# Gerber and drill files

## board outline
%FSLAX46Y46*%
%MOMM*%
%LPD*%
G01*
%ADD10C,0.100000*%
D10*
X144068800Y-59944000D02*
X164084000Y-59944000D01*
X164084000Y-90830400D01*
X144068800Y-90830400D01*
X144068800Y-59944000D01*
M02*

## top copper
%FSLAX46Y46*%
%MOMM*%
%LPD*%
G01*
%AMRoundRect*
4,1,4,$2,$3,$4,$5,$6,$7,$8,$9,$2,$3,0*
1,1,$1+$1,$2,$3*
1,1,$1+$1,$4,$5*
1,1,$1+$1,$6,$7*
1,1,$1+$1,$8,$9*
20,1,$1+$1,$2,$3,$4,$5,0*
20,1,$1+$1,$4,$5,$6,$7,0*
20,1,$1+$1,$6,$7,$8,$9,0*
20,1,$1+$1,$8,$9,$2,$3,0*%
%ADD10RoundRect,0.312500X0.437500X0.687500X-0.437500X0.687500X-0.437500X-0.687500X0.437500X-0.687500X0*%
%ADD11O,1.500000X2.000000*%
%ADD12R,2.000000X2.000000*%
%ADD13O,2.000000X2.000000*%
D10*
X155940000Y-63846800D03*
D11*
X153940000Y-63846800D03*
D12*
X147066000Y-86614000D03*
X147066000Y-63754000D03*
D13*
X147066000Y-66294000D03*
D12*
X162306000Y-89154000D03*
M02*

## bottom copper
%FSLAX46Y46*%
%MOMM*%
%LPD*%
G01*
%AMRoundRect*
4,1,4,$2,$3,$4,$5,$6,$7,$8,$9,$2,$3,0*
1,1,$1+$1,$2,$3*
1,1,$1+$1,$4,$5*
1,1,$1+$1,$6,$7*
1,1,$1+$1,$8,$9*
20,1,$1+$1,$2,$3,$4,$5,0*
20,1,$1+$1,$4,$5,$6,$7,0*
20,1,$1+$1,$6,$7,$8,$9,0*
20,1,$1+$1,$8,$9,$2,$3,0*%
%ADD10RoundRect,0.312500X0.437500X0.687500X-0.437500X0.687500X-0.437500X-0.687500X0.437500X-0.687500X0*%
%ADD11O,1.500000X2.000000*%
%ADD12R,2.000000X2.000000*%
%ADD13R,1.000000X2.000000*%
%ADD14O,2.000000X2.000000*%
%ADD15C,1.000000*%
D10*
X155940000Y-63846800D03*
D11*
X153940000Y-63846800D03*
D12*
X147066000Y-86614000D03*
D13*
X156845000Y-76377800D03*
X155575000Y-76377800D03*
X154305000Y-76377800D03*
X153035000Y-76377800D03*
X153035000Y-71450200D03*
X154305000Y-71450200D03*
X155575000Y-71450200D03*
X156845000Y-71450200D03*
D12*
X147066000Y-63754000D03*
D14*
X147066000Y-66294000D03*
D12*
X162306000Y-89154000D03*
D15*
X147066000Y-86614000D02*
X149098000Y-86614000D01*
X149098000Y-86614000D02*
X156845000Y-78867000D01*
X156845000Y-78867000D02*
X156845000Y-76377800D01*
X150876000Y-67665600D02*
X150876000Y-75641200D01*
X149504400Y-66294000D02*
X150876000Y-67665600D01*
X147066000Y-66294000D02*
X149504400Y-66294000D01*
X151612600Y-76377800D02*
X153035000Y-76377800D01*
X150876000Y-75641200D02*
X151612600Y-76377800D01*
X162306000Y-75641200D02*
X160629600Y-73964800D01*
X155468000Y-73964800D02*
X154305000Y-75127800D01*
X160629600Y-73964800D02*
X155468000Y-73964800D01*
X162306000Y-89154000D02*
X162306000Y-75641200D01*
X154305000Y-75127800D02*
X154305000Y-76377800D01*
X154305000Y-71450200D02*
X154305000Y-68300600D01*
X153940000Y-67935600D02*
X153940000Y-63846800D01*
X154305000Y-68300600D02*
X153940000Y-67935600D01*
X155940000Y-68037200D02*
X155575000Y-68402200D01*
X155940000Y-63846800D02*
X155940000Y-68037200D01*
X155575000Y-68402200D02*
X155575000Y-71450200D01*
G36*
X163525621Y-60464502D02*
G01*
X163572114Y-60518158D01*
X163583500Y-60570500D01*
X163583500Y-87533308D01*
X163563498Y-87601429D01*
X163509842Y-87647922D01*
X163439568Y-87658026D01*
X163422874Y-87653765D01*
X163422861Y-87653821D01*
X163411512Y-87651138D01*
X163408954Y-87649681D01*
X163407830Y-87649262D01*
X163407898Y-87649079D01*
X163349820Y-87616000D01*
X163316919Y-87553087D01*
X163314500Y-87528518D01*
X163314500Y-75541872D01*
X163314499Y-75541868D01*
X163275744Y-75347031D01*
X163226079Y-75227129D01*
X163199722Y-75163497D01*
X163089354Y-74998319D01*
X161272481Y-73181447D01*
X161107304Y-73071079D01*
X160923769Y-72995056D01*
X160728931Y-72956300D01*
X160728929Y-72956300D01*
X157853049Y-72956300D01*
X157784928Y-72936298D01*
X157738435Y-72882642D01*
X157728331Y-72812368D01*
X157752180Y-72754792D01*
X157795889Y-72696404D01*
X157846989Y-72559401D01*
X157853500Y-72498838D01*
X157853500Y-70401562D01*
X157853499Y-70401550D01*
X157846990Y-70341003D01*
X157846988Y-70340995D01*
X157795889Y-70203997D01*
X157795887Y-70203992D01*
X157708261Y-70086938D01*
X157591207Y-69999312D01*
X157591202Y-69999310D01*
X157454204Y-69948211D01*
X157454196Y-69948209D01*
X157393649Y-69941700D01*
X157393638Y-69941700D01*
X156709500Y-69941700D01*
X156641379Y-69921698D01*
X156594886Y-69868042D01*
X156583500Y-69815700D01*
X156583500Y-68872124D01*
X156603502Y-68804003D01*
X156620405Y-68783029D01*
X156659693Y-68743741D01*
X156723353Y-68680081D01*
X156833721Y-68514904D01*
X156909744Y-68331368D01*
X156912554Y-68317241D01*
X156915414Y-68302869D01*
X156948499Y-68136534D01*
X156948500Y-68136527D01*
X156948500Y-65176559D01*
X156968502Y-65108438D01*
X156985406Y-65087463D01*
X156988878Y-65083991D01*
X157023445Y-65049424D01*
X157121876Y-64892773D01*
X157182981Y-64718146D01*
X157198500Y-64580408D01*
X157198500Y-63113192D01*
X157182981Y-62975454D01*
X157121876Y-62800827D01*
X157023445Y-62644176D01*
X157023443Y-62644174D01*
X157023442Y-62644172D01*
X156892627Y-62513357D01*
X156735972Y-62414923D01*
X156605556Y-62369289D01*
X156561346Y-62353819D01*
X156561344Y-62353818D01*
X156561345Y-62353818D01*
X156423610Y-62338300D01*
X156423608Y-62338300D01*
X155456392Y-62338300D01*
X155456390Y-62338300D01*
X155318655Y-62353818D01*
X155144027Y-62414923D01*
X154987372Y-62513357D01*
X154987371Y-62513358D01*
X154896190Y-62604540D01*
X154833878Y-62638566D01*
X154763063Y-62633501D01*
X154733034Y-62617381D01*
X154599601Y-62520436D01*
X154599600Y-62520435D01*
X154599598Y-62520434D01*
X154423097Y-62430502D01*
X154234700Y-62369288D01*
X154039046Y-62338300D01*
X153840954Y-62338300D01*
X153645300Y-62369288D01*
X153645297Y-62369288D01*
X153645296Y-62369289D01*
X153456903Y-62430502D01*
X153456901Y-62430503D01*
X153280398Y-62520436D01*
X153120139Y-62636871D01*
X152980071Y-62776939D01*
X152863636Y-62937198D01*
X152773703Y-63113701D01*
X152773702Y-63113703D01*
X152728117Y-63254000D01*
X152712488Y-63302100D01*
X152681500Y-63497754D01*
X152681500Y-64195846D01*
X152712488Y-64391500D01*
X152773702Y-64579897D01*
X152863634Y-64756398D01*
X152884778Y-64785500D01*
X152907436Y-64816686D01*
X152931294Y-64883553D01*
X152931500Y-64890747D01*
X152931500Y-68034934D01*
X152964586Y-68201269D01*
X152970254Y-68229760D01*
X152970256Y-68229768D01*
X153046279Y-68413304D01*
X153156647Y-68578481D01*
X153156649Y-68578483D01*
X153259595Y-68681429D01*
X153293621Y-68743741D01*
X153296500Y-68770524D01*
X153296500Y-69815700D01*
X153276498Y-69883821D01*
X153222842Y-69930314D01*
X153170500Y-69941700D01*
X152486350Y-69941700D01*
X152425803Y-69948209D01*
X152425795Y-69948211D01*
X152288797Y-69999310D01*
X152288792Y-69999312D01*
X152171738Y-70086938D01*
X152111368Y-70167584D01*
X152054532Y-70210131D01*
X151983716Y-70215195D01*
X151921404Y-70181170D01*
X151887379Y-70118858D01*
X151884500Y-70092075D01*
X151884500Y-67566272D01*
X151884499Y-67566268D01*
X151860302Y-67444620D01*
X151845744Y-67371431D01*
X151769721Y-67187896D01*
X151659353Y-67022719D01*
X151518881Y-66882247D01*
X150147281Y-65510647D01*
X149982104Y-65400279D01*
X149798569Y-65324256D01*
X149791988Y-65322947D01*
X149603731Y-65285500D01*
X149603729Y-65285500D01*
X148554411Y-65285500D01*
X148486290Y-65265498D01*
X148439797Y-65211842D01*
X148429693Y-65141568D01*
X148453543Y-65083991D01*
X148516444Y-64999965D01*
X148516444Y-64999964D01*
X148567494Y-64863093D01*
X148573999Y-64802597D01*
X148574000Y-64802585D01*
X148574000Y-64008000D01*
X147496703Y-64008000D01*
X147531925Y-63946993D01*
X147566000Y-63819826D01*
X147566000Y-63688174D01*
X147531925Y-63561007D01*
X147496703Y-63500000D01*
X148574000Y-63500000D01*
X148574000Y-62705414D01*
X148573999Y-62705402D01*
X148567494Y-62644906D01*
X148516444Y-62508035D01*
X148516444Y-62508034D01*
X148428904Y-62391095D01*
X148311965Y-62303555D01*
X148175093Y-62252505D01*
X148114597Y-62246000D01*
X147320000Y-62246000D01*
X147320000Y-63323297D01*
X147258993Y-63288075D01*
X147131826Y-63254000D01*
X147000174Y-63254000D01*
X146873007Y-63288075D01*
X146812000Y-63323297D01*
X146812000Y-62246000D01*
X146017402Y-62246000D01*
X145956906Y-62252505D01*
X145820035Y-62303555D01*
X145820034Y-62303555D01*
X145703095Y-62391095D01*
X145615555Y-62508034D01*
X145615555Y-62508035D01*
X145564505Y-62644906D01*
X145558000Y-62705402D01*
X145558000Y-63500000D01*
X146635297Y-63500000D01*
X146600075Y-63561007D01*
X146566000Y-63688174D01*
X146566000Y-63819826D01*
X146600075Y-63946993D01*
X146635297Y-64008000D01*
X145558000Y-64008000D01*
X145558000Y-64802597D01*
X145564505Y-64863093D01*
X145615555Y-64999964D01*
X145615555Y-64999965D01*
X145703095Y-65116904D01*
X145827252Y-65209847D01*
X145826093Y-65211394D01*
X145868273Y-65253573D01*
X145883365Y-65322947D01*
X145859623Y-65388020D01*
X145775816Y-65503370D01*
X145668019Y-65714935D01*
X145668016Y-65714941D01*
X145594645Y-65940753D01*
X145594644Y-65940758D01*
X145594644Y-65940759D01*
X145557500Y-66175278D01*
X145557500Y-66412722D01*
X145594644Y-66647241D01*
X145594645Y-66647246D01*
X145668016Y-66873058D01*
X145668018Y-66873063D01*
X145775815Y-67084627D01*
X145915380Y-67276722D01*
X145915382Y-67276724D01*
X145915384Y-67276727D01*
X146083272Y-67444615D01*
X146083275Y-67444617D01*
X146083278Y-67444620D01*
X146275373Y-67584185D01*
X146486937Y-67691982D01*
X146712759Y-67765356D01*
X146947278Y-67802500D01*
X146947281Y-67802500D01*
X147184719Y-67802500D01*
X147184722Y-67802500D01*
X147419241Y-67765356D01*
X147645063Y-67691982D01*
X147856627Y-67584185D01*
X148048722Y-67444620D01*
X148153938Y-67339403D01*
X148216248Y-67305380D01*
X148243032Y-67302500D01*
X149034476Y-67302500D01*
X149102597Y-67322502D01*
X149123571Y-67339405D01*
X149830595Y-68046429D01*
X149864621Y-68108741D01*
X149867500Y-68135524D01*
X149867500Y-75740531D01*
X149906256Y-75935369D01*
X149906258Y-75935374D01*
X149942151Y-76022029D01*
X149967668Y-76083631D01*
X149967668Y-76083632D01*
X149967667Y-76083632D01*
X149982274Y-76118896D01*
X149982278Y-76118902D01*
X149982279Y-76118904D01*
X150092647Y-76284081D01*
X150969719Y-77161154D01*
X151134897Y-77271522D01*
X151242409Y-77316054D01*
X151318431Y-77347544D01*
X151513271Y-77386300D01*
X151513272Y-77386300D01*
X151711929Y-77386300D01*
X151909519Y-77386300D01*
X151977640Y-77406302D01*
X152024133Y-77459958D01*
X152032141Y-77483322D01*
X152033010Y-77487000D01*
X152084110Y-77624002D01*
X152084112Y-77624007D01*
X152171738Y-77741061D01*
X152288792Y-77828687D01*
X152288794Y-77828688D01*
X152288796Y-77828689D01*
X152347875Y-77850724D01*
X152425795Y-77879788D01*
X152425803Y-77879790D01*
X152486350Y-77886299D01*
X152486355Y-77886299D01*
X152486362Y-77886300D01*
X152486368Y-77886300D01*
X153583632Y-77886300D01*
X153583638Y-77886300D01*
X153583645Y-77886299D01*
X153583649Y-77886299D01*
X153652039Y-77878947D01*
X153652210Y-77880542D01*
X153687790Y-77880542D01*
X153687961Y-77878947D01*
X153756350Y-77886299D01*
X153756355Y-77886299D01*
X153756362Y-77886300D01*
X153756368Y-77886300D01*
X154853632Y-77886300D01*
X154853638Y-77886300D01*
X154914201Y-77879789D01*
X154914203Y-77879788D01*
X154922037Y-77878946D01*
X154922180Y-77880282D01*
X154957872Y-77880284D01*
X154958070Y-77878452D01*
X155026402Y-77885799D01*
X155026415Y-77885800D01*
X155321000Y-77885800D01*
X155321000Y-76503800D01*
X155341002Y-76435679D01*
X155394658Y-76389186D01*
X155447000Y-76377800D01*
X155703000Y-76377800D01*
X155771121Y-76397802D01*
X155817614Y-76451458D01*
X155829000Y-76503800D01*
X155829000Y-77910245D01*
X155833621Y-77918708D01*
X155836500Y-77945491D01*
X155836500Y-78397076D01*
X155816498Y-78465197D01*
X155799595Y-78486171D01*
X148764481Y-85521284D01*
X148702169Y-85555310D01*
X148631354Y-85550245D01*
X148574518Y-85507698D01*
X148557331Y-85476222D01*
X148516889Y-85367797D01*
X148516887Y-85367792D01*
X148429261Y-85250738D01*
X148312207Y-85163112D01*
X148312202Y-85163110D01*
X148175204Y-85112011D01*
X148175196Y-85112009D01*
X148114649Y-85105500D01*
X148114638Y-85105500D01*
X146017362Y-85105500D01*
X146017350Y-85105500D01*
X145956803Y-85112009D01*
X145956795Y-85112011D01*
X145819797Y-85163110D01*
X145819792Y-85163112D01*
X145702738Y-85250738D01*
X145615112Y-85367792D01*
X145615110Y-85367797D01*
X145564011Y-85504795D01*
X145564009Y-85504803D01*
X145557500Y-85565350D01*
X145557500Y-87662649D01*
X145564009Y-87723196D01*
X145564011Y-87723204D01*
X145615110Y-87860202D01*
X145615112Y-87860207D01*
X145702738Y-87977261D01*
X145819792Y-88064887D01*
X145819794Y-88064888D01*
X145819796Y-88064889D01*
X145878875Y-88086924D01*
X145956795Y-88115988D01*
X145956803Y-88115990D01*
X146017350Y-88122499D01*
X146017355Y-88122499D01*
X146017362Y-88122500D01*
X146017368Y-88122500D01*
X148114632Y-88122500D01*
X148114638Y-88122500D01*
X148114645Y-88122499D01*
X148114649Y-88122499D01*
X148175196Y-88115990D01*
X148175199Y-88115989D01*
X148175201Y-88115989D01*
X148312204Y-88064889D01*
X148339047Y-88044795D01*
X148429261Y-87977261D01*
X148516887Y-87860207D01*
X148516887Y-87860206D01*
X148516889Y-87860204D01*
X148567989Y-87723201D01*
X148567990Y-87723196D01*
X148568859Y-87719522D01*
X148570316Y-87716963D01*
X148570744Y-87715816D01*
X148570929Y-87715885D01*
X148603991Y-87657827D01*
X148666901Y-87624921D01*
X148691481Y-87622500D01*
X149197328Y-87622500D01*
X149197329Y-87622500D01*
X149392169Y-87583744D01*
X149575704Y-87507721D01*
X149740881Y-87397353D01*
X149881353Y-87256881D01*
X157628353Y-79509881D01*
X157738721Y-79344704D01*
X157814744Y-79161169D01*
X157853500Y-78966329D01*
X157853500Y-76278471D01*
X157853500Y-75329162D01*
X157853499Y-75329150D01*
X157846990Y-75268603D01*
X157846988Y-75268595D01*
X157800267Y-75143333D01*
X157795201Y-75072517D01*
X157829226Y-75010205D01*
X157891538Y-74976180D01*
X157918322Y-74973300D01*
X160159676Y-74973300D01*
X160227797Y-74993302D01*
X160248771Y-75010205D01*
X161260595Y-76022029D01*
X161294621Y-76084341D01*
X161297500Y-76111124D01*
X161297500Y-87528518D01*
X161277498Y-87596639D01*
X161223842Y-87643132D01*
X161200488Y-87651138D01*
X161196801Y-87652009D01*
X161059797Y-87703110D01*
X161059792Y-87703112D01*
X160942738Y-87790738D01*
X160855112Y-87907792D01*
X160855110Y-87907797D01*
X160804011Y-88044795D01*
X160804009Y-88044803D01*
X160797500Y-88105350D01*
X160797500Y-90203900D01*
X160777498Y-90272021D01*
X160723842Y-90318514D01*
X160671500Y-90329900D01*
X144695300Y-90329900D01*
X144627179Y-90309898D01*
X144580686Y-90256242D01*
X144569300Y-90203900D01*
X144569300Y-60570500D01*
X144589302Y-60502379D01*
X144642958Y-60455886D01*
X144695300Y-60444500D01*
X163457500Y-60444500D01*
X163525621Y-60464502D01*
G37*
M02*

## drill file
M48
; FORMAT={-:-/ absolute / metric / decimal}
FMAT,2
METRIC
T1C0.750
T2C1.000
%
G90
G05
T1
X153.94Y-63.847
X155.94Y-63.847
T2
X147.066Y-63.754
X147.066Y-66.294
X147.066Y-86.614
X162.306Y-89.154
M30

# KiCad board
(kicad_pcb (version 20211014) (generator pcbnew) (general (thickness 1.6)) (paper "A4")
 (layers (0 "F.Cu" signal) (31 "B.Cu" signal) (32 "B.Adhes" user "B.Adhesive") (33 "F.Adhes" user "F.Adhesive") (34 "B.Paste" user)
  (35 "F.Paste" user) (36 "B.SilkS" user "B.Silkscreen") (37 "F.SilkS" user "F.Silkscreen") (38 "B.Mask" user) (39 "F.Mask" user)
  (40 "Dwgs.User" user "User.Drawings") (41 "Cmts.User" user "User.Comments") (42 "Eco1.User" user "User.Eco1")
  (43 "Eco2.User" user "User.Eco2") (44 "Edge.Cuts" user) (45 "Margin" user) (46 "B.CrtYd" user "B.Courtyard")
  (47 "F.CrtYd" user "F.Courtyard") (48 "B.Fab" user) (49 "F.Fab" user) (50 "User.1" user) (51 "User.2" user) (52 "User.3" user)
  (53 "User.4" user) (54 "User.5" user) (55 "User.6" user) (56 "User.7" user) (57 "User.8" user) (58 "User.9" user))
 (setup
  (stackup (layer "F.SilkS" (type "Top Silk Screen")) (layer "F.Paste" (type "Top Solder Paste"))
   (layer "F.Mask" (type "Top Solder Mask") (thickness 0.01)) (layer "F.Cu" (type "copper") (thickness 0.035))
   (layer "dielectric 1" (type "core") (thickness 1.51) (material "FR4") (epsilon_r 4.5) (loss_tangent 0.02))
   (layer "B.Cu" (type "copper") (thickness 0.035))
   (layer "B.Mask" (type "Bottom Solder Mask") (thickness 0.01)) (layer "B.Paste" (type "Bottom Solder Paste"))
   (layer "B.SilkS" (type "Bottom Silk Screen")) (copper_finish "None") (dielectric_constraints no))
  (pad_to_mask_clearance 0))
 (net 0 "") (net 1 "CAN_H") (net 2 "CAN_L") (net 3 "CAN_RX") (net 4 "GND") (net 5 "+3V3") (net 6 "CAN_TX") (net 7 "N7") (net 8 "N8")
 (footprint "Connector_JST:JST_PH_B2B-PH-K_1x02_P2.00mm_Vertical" (layer "F.Cu") (at 155.94 63.8468 180)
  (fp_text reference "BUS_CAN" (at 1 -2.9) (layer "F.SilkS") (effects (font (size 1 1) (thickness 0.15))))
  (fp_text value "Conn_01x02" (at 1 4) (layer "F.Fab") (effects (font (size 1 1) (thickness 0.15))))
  (pad "1" thru_hole roundrect locked (at 0 0 180) (size 1.5 2) (drill 0.75) (layers *.Cu *.Mask) (roundrect_rratio 0.208333)
   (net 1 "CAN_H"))
  (pad "2" thru_hole oval locked (at 2 0 180) (size 1.5 2) (drill 0.75) (layers *.Cu *.Mask) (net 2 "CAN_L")))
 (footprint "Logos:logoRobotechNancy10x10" (layer "F.Cu") (at 154.432 74.93)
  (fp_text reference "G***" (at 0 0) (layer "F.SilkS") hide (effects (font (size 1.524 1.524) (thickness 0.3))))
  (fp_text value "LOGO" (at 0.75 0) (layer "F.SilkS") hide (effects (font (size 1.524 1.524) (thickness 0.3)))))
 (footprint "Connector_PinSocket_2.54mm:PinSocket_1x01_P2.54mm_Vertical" (layer "B.Cu") (at 147.066 86.614 180)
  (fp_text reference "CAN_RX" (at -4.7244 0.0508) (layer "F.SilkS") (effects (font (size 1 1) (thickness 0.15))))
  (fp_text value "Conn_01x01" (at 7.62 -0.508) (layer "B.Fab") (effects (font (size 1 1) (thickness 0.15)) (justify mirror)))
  (pad "1" thru_hole rect locked (at 0 0 180) (size 2 2) (drill 1) (layers *.Cu *.Mask) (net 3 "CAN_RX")))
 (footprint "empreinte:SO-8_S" (layer "B.Cu") (at 154.94 73.914 90)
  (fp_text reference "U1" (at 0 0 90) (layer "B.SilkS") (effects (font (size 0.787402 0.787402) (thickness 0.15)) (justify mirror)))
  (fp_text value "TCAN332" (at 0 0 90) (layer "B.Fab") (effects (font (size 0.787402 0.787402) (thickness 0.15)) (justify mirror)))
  (pad "1" smd rect locked (at -2.4638 1.905 90) (size 2 1) (layers "B.Cu" "B.Paste" "B.Mask") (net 3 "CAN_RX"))
  (pad "2" smd rect locked (at -2.4638 0.635 90) (size 2 1) (layers "B.Cu" "B.Paste" "B.Mask") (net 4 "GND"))
  (pad "3" smd rect locked (at -2.4638 -0.635 90) (size 2 1) (layers "B.Cu" "B.Paste" "B.Mask") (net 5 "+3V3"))
  (pad "4" smd rect locked (at -2.4638 -1.905 90) (size 2 1) (layers "B.Cu" "B.Paste" "B.Mask") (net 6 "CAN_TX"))
  (pad "5" smd rect locked (at 2.4638 -1.905 90) (size 2 1) (layers "B.Cu" "B.Paste" "B.Mask") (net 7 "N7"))
  (pad "6" smd rect locked (at 2.4638 -0.635 90) (size 2 1) (layers "B.Cu" "B.Paste" "B.Mask") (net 2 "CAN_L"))
  (pad "7" smd rect locked (at 2.4638 0.635 90) (size 2 1) (layers "B.Cu" "B.Paste" "B.Mask") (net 1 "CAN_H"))
  (pad "8" smd rect locked (at 2.4638 1.905 90) (size 2 1) (layers "B.Cu" "B.Paste" "B.Mask") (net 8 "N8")))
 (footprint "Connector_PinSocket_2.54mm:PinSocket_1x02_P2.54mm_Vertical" (layer "B.Cu") (at 147.066 63.754 180)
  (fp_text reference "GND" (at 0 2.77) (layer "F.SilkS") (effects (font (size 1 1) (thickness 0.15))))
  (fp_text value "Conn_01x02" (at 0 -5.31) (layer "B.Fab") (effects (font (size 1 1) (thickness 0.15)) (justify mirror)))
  (pad "1" thru_hole rect locked (at 0 0 180) (size 2 2) (drill 1) (layers *.Cu *.Mask) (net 4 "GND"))
  (pad "2" thru_hole oval locked (at 0 -2.54 180) (size 2 2) (drill 1) (layers *.Cu *.Mask) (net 6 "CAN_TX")))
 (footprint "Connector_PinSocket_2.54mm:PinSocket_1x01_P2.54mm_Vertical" (layer "B.Cu") (at 162.306 89.154 180)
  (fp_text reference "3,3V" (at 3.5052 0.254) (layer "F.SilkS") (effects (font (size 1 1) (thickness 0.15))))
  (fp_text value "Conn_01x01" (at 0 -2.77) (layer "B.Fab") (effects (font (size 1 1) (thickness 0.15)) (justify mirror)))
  (pad "1" thru_hole rect locked (at 0 0 180) (size 2 2) (drill 1) (layers *.Cu *.Mask) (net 5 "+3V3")))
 (gr_rect (start 144.0688 59.944) (end 164.084 90.8304) (layer "Edge.Cuts") (width 0.1) (fill none))
 (segment (start 147.066 86.614) (end 149.098 86.614) (width 1) (layer "B.Cu") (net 3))
 (segment (start 149.098 86.614) (end 156.845 78.867) (width 1) (layer "B.Cu") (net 3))
 (segment (start 156.845 78.867) (end 156.845 76.3778) (width 1) (layer "B.Cu") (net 3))
 (segment (start 150.876 67.6656) (end 150.876 75.6412) (width 1) (layer "B.Cu") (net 6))
 (segment (start 149.5044 66.294) (end 150.876 67.6656) (width 1) (layer "B.Cu") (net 6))
 (segment (start 147.066 66.294) (end 149.5044 66.294) (width 1) (layer "B.Cu") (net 6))
 (segment (start 151.6126 76.3778) (end 153.035 76.3778) (width 1) (layer "B.Cu") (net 6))
 (segment (start 150.876 75.6412) (end 151.6126 76.3778) (width 1) (layer "B.Cu") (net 6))
 (segment (start 162.306 75.6412) (end 160.6296 73.9648) (width 1) (layer "B.Cu") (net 5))
 (segment (start 155.468 73.9648) (end 154.305 75.1278) (width 1) (layer "B.Cu") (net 5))
 (segment (start 160.6296 73.9648) (end 155.468 73.9648) (width 1) (layer "B.Cu") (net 5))
 (segment (start 162.306 89.154) (end 162.306 75.6412) (width 1) (layer "B.Cu") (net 5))
 (segment (start 154.305 75.1278) (end 154.305 76.3778) (width 1) (layer "B.Cu") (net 5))
 (segment (start 154.305 71.4502) (end 154.305 68.3006) (width 1) (layer "B.Cu") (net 2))
 (segment (start 153.94 67.9356) (end 153.94 63.8468) (width 1) (layer "B.Cu") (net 2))
 (segment (start 154.305 68.3006) (end 153.94 67.9356) (width 1) (layer "B.Cu") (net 2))
 (segment (start 155.94 68.0372) (end 155.575 68.4022) (width 1) (layer "B.Cu") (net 1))
 (segment (start 155.94 63.8468) (end 155.94 68.0372) (width 1) (layer "B.Cu") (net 1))
 (segment (start 155.575 68.4022) (end 155.575 71.4502) (width 1) (layer "B.Cu") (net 1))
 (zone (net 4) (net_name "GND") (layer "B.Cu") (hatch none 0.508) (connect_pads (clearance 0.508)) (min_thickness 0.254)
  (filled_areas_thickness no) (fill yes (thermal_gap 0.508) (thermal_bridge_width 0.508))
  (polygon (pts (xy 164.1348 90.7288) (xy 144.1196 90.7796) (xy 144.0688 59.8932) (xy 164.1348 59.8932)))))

